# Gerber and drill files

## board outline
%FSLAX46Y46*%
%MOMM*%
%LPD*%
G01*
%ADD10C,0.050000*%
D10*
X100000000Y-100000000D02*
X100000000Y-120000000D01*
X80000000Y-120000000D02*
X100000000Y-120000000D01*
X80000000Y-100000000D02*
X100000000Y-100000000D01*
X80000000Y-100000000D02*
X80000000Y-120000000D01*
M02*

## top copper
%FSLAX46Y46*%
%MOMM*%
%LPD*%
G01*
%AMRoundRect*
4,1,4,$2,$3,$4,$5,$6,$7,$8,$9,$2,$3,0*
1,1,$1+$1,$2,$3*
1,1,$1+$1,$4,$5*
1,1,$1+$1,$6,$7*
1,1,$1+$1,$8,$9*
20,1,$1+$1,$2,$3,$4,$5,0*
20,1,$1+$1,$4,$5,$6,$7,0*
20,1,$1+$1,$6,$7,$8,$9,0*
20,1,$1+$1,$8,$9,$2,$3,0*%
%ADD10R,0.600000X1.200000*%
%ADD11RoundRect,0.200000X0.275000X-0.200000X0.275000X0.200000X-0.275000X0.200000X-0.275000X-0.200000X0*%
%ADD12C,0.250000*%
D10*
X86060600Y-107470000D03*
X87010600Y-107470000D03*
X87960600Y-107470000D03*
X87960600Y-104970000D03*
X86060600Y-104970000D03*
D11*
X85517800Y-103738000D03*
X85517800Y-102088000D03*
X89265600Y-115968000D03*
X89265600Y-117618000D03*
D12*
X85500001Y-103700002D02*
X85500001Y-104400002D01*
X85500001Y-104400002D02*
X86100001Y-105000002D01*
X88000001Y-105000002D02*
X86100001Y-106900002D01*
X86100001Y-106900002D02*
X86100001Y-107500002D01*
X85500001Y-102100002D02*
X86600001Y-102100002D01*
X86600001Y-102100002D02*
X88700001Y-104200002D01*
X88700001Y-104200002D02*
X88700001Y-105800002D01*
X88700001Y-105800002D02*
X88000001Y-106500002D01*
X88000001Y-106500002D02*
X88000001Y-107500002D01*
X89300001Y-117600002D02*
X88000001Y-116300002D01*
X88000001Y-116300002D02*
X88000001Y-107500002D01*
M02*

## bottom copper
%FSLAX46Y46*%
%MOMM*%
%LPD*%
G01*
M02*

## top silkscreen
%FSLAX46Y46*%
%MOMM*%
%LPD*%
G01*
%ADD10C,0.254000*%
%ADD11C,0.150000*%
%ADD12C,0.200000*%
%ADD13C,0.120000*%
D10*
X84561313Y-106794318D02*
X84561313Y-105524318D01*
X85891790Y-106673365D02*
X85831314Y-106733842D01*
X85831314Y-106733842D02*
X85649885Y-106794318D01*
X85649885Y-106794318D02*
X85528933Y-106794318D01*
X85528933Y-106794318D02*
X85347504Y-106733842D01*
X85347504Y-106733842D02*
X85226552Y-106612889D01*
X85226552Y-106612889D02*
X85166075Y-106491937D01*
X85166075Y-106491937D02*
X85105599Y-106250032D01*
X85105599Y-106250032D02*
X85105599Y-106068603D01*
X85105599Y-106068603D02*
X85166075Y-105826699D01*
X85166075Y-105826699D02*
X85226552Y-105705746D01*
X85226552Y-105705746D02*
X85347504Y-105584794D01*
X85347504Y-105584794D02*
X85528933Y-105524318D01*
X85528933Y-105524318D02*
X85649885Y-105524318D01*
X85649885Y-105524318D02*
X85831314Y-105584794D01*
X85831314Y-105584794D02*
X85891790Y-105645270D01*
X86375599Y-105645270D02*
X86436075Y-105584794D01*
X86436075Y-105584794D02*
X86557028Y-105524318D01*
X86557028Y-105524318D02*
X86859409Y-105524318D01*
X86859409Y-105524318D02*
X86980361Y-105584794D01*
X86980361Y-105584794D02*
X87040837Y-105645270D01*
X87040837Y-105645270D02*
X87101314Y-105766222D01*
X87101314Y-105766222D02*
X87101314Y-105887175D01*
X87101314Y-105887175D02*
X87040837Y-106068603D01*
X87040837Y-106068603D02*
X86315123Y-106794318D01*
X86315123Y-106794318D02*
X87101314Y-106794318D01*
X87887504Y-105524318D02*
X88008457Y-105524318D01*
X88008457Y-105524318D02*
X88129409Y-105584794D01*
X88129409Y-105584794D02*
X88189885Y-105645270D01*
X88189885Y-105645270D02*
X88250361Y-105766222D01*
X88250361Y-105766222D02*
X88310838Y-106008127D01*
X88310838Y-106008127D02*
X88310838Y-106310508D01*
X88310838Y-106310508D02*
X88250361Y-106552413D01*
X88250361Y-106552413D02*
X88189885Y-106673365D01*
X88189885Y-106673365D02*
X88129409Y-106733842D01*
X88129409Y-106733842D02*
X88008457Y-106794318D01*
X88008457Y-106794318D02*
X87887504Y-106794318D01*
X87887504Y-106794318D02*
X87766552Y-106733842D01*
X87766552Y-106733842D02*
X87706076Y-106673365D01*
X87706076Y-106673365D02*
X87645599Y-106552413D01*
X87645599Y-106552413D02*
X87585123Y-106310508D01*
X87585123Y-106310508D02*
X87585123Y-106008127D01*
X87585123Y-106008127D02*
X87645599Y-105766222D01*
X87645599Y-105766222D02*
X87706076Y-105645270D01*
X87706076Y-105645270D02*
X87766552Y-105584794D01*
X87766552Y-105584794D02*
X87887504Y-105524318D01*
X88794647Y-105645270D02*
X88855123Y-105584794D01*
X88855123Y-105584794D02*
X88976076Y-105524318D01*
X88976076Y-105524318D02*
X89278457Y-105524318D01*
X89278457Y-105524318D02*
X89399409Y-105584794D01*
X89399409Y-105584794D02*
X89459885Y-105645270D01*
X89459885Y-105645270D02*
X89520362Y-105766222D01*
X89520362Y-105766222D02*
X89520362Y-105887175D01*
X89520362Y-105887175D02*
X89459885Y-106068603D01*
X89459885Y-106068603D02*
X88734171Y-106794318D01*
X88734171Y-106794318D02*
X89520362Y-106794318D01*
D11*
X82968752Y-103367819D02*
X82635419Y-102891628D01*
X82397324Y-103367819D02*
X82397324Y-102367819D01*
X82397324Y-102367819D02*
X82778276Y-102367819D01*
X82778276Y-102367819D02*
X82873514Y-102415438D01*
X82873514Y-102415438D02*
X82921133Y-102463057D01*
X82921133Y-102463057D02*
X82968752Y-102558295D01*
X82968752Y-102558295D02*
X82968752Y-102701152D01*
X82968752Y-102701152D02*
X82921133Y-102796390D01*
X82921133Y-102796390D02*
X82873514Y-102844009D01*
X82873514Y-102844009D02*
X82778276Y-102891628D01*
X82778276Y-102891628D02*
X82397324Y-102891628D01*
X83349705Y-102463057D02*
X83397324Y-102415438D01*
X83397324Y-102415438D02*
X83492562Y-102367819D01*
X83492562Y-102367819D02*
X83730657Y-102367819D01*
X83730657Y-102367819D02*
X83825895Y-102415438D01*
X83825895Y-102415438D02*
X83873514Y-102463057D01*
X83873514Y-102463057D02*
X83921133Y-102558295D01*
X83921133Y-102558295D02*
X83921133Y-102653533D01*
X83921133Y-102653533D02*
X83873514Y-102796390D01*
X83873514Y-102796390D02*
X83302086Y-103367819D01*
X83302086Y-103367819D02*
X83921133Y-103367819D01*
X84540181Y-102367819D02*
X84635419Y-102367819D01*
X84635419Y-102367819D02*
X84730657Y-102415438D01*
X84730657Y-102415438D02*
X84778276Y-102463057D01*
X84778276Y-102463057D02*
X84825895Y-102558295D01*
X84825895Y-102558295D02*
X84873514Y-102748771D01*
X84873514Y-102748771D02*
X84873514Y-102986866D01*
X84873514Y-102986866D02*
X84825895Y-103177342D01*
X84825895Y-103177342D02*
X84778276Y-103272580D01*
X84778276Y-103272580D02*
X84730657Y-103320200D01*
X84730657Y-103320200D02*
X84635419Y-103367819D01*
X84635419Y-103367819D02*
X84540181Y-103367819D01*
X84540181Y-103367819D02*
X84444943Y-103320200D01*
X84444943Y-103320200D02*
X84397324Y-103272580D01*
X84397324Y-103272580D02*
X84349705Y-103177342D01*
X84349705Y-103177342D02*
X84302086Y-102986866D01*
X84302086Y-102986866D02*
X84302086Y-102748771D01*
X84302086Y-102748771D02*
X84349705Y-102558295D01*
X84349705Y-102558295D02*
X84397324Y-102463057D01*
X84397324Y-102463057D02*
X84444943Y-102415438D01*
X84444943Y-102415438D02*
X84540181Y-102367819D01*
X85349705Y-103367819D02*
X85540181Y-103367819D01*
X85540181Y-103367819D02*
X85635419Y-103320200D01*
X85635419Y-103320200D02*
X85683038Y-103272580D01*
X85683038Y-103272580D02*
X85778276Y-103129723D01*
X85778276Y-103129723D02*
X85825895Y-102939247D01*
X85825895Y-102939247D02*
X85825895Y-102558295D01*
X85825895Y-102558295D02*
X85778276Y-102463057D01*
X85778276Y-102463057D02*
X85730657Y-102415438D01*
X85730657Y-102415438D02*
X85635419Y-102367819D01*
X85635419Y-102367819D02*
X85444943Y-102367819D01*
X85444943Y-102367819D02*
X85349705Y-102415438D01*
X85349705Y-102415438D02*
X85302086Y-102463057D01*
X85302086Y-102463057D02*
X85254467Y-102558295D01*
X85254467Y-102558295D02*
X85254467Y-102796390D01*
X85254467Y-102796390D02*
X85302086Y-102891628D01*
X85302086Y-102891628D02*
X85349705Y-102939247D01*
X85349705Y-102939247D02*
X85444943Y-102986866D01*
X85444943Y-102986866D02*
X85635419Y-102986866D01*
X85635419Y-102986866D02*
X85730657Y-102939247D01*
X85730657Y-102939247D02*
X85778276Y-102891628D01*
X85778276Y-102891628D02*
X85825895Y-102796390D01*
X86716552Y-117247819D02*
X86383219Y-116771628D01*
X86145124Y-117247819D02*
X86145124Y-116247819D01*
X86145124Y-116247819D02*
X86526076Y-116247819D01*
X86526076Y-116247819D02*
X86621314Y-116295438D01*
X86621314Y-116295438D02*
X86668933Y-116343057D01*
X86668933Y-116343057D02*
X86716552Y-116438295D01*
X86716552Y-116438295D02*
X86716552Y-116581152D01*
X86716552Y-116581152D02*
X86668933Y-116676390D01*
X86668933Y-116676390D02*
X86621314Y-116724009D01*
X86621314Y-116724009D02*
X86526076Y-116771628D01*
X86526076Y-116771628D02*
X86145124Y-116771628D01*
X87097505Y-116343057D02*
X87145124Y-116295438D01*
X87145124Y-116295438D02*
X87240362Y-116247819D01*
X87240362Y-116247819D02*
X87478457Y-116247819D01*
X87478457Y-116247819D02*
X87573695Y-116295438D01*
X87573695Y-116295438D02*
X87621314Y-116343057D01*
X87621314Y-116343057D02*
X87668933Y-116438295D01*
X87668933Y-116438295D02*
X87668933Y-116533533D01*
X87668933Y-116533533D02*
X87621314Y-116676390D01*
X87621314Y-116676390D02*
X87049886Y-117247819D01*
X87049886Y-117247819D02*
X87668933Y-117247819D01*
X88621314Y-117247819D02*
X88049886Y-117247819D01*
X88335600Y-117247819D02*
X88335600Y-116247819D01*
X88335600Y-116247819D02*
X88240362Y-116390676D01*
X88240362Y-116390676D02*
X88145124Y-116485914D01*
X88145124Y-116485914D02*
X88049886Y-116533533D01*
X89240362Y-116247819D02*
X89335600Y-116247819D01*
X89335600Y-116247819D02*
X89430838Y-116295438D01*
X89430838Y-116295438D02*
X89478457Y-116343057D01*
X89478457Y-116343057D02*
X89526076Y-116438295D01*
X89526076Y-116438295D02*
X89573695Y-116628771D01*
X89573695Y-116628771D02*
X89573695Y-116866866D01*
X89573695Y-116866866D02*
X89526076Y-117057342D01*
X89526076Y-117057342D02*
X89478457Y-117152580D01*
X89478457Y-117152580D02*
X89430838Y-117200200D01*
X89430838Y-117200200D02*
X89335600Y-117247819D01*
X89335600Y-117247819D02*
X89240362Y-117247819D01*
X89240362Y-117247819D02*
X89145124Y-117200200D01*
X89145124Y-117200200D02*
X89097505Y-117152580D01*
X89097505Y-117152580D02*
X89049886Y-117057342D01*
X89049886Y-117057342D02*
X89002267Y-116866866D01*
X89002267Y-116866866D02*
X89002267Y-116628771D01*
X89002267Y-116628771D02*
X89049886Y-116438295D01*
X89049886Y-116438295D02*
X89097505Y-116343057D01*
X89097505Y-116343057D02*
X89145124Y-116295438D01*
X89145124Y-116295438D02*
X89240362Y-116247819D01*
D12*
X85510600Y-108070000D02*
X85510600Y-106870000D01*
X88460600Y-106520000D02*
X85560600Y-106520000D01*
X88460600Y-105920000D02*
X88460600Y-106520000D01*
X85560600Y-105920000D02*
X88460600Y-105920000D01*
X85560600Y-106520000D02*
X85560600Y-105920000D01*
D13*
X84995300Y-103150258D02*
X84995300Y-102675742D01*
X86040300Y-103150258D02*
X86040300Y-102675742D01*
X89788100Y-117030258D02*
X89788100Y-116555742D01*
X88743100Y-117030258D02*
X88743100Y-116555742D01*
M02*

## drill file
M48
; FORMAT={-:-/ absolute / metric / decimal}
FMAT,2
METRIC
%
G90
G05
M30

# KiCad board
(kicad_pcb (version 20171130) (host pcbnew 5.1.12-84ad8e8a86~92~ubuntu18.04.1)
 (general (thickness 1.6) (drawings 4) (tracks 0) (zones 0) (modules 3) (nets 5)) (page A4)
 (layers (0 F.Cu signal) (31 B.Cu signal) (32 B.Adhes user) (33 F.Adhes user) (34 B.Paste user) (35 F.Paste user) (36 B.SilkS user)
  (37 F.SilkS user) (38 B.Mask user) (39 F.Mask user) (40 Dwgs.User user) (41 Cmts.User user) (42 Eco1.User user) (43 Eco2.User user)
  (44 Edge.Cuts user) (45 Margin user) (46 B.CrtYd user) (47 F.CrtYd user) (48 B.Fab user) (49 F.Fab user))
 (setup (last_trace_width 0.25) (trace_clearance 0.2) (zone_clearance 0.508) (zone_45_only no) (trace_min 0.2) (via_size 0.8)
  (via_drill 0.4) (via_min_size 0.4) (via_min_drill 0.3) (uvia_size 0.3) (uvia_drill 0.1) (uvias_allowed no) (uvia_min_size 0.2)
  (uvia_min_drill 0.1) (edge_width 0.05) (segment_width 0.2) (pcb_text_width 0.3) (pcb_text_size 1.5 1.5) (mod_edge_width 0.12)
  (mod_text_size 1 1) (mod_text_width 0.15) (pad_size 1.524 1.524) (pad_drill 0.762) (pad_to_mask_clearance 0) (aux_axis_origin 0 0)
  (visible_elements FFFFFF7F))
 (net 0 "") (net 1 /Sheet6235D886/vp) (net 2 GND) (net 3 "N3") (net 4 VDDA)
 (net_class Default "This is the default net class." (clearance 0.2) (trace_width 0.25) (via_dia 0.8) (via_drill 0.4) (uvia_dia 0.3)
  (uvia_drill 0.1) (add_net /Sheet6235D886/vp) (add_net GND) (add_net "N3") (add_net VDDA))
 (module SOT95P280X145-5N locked (layer F.Cu) (at 87.010600 106.220000 90.000000)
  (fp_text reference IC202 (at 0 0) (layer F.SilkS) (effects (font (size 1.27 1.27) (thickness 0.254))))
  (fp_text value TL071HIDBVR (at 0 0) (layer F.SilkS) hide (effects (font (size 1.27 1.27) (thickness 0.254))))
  (fp_line (start -1.85 -1.5) (end -0.65 -1.5) (layer F.SilkS) (width 0.2))
  (fp_line (start -0.3 1.45) (end -0.3 -1.45) (layer F.SilkS) (width 0.2))
  (fp_line (start 0.3 1.45) (end -0.3 1.45) (layer F.SilkS) (width 0.2))
  (fp_line (start 0.3 -1.45) (end 0.3 1.45) (layer F.SilkS) (width 0.2))
  (fp_line (start -0.3 -1.45) (end 0.3 -1.45) (layer F.SilkS) (width 0.2))
  (pad 1 smd rect (at -1.25 -0.95 180.000000) (size 0.6 1.2) (layers F.Cu F.Mask F.Paste) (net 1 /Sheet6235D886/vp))
  (pad 2 smd rect (at -1.25 0 180.000000) (size 0.6 1.2) (layers F.Cu F.Mask F.Paste) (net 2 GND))
  (pad 3 smd rect (at -1.25 0.95 180.000000) (size 0.6 1.2) (layers F.Cu F.Mask F.Paste) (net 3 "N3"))
  (pad 4 smd rect (at 1.25 0.95 180.000000) (size 0.6 1.2) (layers F.Cu F.Mask F.Paste) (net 1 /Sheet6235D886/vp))
  (pad 5 smd rect (at 1.25 -0.95 180.000000) (size 0.6 1.2) (layers F.Cu F.Mask F.Paste) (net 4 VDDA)))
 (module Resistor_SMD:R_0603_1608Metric (layer F.Cu) (at 85.517800 102.913000 90.000000)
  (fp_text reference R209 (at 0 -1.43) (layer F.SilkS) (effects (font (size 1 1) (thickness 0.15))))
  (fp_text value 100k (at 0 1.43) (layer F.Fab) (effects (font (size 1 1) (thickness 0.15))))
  (fp_line (start -0.237258 -0.5225) (end 0.237258 -0.5225) (layer F.SilkS) (width 0.12))
  (fp_line (start -0.237258 0.5225) (end 0.237258 0.5225) (layer F.SilkS) (width 0.12))
  (pad 1 smd roundrect (at -0.825 0 90.000000) (size 0.8 0.95) (layers F.Cu F.Mask F.Paste) (roundrect_rratio 0.25) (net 4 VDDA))
  (pad 2 smd roundrect (at 0.825 0 90.000000) (size 0.8 0.95) (layers F.Cu F.Mask F.Paste) (roundrect_rratio 0.25) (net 3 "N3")))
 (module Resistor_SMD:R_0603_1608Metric (layer F.Cu) (at 89.265600 116.793000 90.000000)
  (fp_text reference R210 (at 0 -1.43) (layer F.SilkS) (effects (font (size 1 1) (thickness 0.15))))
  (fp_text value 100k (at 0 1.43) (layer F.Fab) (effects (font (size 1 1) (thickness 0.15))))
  (fp_line (start -0.237258 0.5225) (end 0.237258 0.5225) (layer F.SilkS) (width 0.12))
  (fp_line (start -0.237258 -0.5225) (end 0.237258 -0.5225) (layer F.SilkS) (width 0.12))
  (pad 2 smd roundrect (at 0.825 0 90.000000) (size 0.8 0.95) (layers F.Cu F.Mask F.Paste) (roundrect_rratio 0.25) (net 2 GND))
  (pad 1 smd roundrect (at -0.825 0 90.000000) (size 0.8 0.95) (layers F.Cu F.Mask F.Paste) (roundrect_rratio 0.25) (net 3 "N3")))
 (gr_line (start 100 100) (end 100 120) (layer Edge.Cuts) (width 0.05))
 (gr_line (start 80 120) (end 100 120) (layer Edge.Cuts) (width 0.05))
 (gr_line (start 80 100) (end 100 100) (layer Edge.Cuts) (width 0.05))
 (gr_line (start 80 100) (end 80 120) (layer Edge.Cuts) (width 0.05))
 (segment (start 85.500001 103.700002) (end 85.500001 104.400002) (width 0.250000) (layer F.Cu) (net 4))
 (segment (start 85.500001 104.400002) (end 86.100001 105.000002) (width 0.250000) (layer F.Cu) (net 4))
 (segment (start 88.000001 105.000002) (end 86.100001 106.900002) (width 0.250000) (layer F.Cu) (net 1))
 (segment (start 86.100001 106.900002) (end 86.100001 107.500002) (width 0.250000) (layer F.Cu) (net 1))
 (segment (start 85.500001 102.100002) (end 86.600001 102.100002) (width 0.250000) (layer F.Cu) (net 3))
 (segment (start 86.600001 102.100002) (end 88.700001 104.200002) (width 0.250000) (layer F.Cu) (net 3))
 (segment (start 88.700001 104.200002) (end 88.700001 105.800002) (width 0.250000) (layer F.Cu) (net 3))
 (segment (start 88.700001 105.800002) (end 88.000001 106.500002) (width 0.250000) (layer F.Cu) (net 3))
 (segment (start 88.000001 106.500002) (end 88.000001 107.500002) (width 0.250000) (layer F.Cu) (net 3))
 (segment (start 89.300001 117.600002) (end 88.000001 116.300002) (width 0.250000) (layer F.Cu) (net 3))
 (segment (start 88.000001 116.300002) (end 88.000001 107.500002) (width 0.250000) (layer F.Cu) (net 3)))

